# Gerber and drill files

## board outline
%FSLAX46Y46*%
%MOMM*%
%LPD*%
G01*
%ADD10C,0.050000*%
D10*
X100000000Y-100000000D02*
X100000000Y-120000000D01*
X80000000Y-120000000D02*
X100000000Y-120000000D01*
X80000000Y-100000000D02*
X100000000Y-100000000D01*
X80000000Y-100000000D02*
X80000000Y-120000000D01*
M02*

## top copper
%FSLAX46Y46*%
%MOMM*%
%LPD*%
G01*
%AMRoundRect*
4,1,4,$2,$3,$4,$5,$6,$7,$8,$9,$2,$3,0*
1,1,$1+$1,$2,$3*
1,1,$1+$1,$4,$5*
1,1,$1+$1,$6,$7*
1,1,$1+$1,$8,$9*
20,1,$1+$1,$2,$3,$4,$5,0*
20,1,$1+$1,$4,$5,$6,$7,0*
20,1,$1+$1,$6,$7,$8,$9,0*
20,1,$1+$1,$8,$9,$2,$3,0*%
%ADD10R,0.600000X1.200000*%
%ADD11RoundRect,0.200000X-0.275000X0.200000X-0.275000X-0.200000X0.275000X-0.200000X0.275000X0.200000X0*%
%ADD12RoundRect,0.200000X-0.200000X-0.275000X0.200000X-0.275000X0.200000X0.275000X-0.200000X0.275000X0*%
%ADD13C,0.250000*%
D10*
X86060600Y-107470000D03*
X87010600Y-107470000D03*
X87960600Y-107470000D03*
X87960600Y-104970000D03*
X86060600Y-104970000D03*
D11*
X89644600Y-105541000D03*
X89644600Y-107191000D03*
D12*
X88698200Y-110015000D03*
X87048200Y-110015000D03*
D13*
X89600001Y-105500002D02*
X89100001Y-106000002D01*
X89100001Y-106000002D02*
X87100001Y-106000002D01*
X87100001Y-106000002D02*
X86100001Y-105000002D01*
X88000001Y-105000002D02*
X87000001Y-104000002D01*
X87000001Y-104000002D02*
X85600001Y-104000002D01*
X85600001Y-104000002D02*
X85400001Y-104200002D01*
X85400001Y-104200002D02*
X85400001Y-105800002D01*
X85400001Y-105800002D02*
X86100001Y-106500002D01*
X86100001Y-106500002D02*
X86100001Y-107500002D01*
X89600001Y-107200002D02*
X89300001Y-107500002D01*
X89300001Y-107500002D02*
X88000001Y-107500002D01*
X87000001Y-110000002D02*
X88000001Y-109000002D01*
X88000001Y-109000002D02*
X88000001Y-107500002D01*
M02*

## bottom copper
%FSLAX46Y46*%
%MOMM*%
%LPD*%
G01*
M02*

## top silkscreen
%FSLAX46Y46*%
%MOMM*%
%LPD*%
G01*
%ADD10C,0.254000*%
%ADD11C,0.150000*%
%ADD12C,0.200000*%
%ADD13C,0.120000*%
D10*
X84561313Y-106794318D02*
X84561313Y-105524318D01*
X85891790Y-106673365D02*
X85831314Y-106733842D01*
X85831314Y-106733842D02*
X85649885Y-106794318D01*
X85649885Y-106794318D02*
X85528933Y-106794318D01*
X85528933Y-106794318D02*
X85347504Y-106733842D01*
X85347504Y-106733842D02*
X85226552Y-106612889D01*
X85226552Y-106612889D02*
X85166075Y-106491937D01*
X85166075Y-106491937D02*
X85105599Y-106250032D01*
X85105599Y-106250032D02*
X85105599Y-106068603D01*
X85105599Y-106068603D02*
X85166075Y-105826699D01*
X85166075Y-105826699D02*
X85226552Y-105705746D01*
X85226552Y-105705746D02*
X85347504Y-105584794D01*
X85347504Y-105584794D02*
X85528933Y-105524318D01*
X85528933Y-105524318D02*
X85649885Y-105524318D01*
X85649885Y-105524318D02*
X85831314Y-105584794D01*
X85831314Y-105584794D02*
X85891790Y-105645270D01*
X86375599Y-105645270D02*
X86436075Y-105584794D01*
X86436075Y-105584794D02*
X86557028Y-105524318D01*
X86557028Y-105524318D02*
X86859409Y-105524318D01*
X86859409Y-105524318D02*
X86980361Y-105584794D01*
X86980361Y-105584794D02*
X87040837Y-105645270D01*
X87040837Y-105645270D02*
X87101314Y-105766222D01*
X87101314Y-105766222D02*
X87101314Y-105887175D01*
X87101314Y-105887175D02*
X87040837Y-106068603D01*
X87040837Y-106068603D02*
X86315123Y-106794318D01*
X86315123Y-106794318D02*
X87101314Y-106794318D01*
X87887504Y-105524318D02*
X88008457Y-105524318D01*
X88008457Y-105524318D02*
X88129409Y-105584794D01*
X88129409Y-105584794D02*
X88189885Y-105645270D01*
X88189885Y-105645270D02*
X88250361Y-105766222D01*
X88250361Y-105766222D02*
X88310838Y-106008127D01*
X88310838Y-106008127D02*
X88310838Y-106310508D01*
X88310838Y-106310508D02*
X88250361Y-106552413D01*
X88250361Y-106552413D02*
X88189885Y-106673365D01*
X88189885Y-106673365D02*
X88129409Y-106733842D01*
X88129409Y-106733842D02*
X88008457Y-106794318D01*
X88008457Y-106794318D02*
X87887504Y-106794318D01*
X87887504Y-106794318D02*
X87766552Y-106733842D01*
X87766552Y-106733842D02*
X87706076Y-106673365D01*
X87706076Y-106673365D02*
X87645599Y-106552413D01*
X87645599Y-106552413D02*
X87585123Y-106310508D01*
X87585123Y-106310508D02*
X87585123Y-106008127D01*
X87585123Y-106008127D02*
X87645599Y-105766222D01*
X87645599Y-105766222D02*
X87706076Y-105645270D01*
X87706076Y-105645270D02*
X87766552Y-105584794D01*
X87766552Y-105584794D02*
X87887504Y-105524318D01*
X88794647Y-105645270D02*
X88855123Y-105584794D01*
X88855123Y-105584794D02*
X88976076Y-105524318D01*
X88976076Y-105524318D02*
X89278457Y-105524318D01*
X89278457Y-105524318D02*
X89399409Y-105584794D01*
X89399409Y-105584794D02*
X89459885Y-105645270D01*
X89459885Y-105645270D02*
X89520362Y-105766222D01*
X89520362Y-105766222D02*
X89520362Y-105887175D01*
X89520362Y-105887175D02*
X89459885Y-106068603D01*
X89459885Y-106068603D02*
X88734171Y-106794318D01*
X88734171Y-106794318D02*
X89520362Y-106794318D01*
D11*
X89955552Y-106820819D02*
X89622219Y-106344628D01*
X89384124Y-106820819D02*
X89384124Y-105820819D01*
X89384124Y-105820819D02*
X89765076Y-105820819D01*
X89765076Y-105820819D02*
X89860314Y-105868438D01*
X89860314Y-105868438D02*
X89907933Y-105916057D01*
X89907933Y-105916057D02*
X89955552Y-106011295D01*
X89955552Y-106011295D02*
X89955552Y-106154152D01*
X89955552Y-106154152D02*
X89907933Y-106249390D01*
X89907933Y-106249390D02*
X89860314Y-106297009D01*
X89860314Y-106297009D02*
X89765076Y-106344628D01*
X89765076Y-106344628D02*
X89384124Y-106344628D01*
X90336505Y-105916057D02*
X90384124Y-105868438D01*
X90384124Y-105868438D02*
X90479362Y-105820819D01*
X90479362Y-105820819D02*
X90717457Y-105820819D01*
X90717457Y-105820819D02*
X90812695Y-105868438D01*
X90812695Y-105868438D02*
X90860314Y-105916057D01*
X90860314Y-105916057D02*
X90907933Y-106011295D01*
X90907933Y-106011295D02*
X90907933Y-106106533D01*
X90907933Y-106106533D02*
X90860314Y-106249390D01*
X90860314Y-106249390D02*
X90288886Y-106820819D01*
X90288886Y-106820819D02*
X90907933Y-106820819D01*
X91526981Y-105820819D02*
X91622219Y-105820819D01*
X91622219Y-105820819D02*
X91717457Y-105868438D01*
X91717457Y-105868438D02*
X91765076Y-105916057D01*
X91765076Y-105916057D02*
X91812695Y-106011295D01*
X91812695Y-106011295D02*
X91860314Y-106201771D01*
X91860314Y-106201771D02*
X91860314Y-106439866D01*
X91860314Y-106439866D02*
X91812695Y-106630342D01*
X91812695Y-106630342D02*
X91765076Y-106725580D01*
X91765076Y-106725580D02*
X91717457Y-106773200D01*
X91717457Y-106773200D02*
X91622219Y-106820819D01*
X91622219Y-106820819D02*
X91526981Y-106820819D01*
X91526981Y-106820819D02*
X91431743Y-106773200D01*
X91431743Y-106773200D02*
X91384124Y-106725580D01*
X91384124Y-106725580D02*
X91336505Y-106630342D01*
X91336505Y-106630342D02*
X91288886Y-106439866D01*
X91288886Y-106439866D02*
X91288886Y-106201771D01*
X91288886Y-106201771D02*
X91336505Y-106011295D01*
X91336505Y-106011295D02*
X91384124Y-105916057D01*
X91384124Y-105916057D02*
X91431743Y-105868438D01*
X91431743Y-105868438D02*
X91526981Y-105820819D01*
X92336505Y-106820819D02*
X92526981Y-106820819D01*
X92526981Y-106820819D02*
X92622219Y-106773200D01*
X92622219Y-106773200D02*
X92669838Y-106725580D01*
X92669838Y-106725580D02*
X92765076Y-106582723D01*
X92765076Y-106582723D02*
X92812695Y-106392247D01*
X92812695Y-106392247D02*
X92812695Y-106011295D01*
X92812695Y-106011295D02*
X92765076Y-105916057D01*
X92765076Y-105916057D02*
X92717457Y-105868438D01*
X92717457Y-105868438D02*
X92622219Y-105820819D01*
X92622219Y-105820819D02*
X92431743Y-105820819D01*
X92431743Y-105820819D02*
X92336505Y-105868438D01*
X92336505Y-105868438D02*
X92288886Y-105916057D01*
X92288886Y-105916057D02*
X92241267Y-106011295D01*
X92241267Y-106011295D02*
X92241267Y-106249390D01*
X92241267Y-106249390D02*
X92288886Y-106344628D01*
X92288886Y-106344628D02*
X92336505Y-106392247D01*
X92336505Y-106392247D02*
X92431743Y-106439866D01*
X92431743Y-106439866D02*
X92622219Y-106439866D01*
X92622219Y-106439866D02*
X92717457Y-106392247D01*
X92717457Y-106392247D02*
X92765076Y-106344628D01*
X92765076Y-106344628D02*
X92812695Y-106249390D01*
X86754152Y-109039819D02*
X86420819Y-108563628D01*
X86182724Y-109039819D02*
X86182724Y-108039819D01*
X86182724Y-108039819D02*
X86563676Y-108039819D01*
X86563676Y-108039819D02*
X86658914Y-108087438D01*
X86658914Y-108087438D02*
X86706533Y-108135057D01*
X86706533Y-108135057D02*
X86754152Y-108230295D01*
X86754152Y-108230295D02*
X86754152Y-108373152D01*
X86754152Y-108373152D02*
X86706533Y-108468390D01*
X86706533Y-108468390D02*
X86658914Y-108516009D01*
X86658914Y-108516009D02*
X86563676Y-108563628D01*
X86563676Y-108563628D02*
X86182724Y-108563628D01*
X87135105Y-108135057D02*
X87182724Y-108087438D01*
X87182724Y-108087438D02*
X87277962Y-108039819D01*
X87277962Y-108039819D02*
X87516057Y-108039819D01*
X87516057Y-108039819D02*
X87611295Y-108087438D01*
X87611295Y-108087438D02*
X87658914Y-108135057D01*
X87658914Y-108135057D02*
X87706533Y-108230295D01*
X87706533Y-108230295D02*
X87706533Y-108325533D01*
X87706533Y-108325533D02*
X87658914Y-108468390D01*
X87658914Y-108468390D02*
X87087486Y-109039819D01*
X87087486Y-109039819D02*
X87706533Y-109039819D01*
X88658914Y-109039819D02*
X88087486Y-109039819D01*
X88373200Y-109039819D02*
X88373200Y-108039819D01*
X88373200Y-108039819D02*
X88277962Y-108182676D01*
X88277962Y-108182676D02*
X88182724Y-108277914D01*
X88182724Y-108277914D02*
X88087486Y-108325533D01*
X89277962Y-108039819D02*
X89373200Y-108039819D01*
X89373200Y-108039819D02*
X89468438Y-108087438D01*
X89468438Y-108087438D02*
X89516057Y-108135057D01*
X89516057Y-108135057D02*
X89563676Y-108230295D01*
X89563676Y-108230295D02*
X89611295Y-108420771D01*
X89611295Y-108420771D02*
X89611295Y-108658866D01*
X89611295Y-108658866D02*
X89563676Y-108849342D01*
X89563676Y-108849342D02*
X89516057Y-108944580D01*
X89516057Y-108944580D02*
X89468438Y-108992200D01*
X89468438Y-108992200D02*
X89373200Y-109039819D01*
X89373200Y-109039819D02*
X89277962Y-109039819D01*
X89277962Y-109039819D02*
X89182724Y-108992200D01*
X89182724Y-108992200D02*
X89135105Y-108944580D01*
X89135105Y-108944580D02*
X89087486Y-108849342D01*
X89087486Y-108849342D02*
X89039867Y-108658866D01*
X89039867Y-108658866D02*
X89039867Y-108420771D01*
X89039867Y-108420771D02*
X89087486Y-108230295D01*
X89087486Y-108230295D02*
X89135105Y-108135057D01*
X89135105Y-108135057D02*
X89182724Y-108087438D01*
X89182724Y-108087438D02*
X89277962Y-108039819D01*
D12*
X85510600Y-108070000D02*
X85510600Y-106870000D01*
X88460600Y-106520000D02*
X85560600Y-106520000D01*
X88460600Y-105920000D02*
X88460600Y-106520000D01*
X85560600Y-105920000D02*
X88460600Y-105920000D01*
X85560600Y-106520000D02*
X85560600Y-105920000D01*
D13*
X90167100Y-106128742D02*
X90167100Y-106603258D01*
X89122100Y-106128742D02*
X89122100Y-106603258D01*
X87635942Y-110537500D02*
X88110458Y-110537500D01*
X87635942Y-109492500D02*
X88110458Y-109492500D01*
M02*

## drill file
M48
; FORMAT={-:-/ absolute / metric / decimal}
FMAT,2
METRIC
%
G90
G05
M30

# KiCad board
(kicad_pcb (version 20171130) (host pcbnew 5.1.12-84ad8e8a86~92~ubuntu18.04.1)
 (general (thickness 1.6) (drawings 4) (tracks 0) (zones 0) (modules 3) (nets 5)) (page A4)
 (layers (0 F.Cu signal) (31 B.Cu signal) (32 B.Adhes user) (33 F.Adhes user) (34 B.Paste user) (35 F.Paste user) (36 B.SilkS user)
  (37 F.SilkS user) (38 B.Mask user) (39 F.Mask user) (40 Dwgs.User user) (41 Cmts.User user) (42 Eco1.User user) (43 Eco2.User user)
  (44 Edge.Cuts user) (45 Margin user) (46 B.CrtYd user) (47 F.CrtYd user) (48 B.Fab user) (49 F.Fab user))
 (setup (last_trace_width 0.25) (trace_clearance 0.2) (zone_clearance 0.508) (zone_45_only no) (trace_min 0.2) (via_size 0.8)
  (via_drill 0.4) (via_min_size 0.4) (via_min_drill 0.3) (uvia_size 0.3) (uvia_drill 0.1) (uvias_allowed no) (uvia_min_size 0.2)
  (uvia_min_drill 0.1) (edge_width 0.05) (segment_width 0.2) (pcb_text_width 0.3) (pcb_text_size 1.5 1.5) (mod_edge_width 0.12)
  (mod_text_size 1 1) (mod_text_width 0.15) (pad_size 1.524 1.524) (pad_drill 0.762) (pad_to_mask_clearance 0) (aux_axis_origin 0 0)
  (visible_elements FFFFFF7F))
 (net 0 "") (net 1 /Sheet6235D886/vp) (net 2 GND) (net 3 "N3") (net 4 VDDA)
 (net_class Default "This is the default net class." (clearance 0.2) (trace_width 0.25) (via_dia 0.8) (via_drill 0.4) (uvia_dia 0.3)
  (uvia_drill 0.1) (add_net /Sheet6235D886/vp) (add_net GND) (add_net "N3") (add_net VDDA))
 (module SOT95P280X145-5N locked (layer F.Cu) (at 87.010600 106.220000 90.000000)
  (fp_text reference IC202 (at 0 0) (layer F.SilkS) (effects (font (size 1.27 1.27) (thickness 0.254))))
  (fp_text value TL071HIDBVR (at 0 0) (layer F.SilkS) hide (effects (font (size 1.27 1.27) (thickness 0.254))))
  (fp_line (start -1.85 -1.5) (end -0.65 -1.5) (layer F.SilkS) (width 0.2))
  (fp_line (start -0.3 1.45) (end -0.3 -1.45) (layer F.SilkS) (width 0.2))
  (fp_line (start 0.3 1.45) (end -0.3 1.45) (layer F.SilkS) (width 0.2))
  (fp_line (start 0.3 -1.45) (end 0.3 1.45) (layer F.SilkS) (width 0.2))
  (fp_line (start -0.3 -1.45) (end 0.3 -1.45) (layer F.SilkS) (width 0.2))
  (pad 1 smd rect (at -1.25 -0.95 180.000000) (size 0.6 1.2) (layers F.Cu F.Mask F.Paste) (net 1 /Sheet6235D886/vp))
  (pad 2 smd rect (at -1.25 0 180.000000) (size 0.6 1.2) (layers F.Cu F.Mask F.Paste) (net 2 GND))
  (pad 3 smd rect (at -1.25 0.95 180.000000) (size 0.6 1.2) (layers F.Cu F.Mask F.Paste) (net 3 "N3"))
  (pad 4 smd rect (at 1.25 0.95 180.000000) (size 0.6 1.2) (layers F.Cu F.Mask F.Paste) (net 1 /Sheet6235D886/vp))
  (pad 5 smd rect (at 1.25 -0.95 180.000000) (size 0.6 1.2) (layers F.Cu F.Mask F.Paste) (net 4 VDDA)))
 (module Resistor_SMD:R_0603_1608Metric (layer F.Cu) (at 89.644600 106.366000 270.000000)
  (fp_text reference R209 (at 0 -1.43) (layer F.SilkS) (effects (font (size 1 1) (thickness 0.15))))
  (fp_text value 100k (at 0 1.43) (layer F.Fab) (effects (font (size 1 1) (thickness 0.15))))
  (fp_line (start -0.237258 -0.5225) (end 0.237258 -0.5225) (layer F.SilkS) (width 0.12))
  (fp_line (start -0.237258 0.5225) (end 0.237258 0.5225) (layer F.SilkS) (width 0.12))
  (pad 1 smd roundrect (at -0.825 0 270.000000) (size 0.8 0.95) (layers F.Cu F.Mask F.Paste) (roundrect_rratio 0.25) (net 4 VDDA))
  (pad 2 smd roundrect (at 0.825 0 270.000000) (size 0.8 0.95) (layers F.Cu F.Mask F.Paste) (roundrect_rratio 0.25) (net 3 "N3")))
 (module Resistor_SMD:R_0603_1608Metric (layer F.Cu) (at 87.873200 110.015000)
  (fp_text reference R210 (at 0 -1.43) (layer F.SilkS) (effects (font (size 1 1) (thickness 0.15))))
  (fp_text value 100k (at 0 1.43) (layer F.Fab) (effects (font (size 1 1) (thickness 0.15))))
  (fp_line (start -0.237258 0.5225) (end 0.237258 0.5225) (layer F.SilkS) (width 0.12))
  (fp_line (start -0.237258 -0.5225) (end 0.237258 -0.5225) (layer F.SilkS) (width 0.12))
  (pad 2 smd roundrect (at 0.825 0) (size 0.8 0.95) (layers F.Cu F.Mask F.Paste) (roundrect_rratio 0.25) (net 2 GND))
  (pad 1 smd roundrect (at -0.825 0) (size 0.8 0.95) (layers F.Cu F.Mask F.Paste) (roundrect_rratio 0.25) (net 3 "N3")))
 (gr_line (start 100 100) (end 100 120) (layer Edge.Cuts) (width 0.05))
 (gr_line (start 80 120) (end 100 120) (layer Edge.Cuts) (width 0.05))
 (gr_line (start 80 100) (end 100 100) (layer Edge.Cuts) (width 0.05))
 (gr_line (start 80 100) (end 80 120) (layer Edge.Cuts) (width 0.05))
 (segment (start 89.600001 105.500002) (end 89.100001 106.000002) (width 0.250000) (layer F.Cu) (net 4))
 (segment (start 89.100001 106.000002) (end 87.100001 106.000002) (width 0.250000) (layer F.Cu) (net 4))
 (segment (start 87.100001 106.000002) (end 86.100001 105.000002) (width 0.250000) (layer F.Cu) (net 4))
 (segment (start 88.000001 105.000002) (end 87.000001 104.000002) (width 0.250000) (layer F.Cu) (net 1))
 (segment (start 87.000001 104.000002) (end 85.600001 104.000002) (width 0.250000) (layer F.Cu) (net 1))
 (segment (start 85.600001 104.000002) (end 85.400001 104.200002) (width 0.250000) (layer F.Cu) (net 1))
 (segment (start 85.400001 104.200002) (end 85.400001 105.800002) (width 0.250000) (layer F.Cu) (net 1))
 (segment (start 85.400001 105.800002) (end 86.100001 106.500002) (width 0.250000) (layer F.Cu) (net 1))
 (segment (start 86.100001 106.500002) (end 86.100001 107.500002) (width 0.250000) (layer F.Cu) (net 1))
 (segment (start 89.600001 107.200002) (end 89.300001 107.500002) (width 0.250000) (layer F.Cu) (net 3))
 (segment (start 89.300001 107.500002) (end 88.000001 107.500002) (width 0.250000) (layer F.Cu) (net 3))
 (segment (start 87.000001 110.000002) (end 88.000001 109.000002) (width 0.250000) (layer F.Cu) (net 3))
 (segment (start 88.000001 109.000002) (end 88.000001 107.500002) (width 0.250000) (layer F.Cu) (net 3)))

